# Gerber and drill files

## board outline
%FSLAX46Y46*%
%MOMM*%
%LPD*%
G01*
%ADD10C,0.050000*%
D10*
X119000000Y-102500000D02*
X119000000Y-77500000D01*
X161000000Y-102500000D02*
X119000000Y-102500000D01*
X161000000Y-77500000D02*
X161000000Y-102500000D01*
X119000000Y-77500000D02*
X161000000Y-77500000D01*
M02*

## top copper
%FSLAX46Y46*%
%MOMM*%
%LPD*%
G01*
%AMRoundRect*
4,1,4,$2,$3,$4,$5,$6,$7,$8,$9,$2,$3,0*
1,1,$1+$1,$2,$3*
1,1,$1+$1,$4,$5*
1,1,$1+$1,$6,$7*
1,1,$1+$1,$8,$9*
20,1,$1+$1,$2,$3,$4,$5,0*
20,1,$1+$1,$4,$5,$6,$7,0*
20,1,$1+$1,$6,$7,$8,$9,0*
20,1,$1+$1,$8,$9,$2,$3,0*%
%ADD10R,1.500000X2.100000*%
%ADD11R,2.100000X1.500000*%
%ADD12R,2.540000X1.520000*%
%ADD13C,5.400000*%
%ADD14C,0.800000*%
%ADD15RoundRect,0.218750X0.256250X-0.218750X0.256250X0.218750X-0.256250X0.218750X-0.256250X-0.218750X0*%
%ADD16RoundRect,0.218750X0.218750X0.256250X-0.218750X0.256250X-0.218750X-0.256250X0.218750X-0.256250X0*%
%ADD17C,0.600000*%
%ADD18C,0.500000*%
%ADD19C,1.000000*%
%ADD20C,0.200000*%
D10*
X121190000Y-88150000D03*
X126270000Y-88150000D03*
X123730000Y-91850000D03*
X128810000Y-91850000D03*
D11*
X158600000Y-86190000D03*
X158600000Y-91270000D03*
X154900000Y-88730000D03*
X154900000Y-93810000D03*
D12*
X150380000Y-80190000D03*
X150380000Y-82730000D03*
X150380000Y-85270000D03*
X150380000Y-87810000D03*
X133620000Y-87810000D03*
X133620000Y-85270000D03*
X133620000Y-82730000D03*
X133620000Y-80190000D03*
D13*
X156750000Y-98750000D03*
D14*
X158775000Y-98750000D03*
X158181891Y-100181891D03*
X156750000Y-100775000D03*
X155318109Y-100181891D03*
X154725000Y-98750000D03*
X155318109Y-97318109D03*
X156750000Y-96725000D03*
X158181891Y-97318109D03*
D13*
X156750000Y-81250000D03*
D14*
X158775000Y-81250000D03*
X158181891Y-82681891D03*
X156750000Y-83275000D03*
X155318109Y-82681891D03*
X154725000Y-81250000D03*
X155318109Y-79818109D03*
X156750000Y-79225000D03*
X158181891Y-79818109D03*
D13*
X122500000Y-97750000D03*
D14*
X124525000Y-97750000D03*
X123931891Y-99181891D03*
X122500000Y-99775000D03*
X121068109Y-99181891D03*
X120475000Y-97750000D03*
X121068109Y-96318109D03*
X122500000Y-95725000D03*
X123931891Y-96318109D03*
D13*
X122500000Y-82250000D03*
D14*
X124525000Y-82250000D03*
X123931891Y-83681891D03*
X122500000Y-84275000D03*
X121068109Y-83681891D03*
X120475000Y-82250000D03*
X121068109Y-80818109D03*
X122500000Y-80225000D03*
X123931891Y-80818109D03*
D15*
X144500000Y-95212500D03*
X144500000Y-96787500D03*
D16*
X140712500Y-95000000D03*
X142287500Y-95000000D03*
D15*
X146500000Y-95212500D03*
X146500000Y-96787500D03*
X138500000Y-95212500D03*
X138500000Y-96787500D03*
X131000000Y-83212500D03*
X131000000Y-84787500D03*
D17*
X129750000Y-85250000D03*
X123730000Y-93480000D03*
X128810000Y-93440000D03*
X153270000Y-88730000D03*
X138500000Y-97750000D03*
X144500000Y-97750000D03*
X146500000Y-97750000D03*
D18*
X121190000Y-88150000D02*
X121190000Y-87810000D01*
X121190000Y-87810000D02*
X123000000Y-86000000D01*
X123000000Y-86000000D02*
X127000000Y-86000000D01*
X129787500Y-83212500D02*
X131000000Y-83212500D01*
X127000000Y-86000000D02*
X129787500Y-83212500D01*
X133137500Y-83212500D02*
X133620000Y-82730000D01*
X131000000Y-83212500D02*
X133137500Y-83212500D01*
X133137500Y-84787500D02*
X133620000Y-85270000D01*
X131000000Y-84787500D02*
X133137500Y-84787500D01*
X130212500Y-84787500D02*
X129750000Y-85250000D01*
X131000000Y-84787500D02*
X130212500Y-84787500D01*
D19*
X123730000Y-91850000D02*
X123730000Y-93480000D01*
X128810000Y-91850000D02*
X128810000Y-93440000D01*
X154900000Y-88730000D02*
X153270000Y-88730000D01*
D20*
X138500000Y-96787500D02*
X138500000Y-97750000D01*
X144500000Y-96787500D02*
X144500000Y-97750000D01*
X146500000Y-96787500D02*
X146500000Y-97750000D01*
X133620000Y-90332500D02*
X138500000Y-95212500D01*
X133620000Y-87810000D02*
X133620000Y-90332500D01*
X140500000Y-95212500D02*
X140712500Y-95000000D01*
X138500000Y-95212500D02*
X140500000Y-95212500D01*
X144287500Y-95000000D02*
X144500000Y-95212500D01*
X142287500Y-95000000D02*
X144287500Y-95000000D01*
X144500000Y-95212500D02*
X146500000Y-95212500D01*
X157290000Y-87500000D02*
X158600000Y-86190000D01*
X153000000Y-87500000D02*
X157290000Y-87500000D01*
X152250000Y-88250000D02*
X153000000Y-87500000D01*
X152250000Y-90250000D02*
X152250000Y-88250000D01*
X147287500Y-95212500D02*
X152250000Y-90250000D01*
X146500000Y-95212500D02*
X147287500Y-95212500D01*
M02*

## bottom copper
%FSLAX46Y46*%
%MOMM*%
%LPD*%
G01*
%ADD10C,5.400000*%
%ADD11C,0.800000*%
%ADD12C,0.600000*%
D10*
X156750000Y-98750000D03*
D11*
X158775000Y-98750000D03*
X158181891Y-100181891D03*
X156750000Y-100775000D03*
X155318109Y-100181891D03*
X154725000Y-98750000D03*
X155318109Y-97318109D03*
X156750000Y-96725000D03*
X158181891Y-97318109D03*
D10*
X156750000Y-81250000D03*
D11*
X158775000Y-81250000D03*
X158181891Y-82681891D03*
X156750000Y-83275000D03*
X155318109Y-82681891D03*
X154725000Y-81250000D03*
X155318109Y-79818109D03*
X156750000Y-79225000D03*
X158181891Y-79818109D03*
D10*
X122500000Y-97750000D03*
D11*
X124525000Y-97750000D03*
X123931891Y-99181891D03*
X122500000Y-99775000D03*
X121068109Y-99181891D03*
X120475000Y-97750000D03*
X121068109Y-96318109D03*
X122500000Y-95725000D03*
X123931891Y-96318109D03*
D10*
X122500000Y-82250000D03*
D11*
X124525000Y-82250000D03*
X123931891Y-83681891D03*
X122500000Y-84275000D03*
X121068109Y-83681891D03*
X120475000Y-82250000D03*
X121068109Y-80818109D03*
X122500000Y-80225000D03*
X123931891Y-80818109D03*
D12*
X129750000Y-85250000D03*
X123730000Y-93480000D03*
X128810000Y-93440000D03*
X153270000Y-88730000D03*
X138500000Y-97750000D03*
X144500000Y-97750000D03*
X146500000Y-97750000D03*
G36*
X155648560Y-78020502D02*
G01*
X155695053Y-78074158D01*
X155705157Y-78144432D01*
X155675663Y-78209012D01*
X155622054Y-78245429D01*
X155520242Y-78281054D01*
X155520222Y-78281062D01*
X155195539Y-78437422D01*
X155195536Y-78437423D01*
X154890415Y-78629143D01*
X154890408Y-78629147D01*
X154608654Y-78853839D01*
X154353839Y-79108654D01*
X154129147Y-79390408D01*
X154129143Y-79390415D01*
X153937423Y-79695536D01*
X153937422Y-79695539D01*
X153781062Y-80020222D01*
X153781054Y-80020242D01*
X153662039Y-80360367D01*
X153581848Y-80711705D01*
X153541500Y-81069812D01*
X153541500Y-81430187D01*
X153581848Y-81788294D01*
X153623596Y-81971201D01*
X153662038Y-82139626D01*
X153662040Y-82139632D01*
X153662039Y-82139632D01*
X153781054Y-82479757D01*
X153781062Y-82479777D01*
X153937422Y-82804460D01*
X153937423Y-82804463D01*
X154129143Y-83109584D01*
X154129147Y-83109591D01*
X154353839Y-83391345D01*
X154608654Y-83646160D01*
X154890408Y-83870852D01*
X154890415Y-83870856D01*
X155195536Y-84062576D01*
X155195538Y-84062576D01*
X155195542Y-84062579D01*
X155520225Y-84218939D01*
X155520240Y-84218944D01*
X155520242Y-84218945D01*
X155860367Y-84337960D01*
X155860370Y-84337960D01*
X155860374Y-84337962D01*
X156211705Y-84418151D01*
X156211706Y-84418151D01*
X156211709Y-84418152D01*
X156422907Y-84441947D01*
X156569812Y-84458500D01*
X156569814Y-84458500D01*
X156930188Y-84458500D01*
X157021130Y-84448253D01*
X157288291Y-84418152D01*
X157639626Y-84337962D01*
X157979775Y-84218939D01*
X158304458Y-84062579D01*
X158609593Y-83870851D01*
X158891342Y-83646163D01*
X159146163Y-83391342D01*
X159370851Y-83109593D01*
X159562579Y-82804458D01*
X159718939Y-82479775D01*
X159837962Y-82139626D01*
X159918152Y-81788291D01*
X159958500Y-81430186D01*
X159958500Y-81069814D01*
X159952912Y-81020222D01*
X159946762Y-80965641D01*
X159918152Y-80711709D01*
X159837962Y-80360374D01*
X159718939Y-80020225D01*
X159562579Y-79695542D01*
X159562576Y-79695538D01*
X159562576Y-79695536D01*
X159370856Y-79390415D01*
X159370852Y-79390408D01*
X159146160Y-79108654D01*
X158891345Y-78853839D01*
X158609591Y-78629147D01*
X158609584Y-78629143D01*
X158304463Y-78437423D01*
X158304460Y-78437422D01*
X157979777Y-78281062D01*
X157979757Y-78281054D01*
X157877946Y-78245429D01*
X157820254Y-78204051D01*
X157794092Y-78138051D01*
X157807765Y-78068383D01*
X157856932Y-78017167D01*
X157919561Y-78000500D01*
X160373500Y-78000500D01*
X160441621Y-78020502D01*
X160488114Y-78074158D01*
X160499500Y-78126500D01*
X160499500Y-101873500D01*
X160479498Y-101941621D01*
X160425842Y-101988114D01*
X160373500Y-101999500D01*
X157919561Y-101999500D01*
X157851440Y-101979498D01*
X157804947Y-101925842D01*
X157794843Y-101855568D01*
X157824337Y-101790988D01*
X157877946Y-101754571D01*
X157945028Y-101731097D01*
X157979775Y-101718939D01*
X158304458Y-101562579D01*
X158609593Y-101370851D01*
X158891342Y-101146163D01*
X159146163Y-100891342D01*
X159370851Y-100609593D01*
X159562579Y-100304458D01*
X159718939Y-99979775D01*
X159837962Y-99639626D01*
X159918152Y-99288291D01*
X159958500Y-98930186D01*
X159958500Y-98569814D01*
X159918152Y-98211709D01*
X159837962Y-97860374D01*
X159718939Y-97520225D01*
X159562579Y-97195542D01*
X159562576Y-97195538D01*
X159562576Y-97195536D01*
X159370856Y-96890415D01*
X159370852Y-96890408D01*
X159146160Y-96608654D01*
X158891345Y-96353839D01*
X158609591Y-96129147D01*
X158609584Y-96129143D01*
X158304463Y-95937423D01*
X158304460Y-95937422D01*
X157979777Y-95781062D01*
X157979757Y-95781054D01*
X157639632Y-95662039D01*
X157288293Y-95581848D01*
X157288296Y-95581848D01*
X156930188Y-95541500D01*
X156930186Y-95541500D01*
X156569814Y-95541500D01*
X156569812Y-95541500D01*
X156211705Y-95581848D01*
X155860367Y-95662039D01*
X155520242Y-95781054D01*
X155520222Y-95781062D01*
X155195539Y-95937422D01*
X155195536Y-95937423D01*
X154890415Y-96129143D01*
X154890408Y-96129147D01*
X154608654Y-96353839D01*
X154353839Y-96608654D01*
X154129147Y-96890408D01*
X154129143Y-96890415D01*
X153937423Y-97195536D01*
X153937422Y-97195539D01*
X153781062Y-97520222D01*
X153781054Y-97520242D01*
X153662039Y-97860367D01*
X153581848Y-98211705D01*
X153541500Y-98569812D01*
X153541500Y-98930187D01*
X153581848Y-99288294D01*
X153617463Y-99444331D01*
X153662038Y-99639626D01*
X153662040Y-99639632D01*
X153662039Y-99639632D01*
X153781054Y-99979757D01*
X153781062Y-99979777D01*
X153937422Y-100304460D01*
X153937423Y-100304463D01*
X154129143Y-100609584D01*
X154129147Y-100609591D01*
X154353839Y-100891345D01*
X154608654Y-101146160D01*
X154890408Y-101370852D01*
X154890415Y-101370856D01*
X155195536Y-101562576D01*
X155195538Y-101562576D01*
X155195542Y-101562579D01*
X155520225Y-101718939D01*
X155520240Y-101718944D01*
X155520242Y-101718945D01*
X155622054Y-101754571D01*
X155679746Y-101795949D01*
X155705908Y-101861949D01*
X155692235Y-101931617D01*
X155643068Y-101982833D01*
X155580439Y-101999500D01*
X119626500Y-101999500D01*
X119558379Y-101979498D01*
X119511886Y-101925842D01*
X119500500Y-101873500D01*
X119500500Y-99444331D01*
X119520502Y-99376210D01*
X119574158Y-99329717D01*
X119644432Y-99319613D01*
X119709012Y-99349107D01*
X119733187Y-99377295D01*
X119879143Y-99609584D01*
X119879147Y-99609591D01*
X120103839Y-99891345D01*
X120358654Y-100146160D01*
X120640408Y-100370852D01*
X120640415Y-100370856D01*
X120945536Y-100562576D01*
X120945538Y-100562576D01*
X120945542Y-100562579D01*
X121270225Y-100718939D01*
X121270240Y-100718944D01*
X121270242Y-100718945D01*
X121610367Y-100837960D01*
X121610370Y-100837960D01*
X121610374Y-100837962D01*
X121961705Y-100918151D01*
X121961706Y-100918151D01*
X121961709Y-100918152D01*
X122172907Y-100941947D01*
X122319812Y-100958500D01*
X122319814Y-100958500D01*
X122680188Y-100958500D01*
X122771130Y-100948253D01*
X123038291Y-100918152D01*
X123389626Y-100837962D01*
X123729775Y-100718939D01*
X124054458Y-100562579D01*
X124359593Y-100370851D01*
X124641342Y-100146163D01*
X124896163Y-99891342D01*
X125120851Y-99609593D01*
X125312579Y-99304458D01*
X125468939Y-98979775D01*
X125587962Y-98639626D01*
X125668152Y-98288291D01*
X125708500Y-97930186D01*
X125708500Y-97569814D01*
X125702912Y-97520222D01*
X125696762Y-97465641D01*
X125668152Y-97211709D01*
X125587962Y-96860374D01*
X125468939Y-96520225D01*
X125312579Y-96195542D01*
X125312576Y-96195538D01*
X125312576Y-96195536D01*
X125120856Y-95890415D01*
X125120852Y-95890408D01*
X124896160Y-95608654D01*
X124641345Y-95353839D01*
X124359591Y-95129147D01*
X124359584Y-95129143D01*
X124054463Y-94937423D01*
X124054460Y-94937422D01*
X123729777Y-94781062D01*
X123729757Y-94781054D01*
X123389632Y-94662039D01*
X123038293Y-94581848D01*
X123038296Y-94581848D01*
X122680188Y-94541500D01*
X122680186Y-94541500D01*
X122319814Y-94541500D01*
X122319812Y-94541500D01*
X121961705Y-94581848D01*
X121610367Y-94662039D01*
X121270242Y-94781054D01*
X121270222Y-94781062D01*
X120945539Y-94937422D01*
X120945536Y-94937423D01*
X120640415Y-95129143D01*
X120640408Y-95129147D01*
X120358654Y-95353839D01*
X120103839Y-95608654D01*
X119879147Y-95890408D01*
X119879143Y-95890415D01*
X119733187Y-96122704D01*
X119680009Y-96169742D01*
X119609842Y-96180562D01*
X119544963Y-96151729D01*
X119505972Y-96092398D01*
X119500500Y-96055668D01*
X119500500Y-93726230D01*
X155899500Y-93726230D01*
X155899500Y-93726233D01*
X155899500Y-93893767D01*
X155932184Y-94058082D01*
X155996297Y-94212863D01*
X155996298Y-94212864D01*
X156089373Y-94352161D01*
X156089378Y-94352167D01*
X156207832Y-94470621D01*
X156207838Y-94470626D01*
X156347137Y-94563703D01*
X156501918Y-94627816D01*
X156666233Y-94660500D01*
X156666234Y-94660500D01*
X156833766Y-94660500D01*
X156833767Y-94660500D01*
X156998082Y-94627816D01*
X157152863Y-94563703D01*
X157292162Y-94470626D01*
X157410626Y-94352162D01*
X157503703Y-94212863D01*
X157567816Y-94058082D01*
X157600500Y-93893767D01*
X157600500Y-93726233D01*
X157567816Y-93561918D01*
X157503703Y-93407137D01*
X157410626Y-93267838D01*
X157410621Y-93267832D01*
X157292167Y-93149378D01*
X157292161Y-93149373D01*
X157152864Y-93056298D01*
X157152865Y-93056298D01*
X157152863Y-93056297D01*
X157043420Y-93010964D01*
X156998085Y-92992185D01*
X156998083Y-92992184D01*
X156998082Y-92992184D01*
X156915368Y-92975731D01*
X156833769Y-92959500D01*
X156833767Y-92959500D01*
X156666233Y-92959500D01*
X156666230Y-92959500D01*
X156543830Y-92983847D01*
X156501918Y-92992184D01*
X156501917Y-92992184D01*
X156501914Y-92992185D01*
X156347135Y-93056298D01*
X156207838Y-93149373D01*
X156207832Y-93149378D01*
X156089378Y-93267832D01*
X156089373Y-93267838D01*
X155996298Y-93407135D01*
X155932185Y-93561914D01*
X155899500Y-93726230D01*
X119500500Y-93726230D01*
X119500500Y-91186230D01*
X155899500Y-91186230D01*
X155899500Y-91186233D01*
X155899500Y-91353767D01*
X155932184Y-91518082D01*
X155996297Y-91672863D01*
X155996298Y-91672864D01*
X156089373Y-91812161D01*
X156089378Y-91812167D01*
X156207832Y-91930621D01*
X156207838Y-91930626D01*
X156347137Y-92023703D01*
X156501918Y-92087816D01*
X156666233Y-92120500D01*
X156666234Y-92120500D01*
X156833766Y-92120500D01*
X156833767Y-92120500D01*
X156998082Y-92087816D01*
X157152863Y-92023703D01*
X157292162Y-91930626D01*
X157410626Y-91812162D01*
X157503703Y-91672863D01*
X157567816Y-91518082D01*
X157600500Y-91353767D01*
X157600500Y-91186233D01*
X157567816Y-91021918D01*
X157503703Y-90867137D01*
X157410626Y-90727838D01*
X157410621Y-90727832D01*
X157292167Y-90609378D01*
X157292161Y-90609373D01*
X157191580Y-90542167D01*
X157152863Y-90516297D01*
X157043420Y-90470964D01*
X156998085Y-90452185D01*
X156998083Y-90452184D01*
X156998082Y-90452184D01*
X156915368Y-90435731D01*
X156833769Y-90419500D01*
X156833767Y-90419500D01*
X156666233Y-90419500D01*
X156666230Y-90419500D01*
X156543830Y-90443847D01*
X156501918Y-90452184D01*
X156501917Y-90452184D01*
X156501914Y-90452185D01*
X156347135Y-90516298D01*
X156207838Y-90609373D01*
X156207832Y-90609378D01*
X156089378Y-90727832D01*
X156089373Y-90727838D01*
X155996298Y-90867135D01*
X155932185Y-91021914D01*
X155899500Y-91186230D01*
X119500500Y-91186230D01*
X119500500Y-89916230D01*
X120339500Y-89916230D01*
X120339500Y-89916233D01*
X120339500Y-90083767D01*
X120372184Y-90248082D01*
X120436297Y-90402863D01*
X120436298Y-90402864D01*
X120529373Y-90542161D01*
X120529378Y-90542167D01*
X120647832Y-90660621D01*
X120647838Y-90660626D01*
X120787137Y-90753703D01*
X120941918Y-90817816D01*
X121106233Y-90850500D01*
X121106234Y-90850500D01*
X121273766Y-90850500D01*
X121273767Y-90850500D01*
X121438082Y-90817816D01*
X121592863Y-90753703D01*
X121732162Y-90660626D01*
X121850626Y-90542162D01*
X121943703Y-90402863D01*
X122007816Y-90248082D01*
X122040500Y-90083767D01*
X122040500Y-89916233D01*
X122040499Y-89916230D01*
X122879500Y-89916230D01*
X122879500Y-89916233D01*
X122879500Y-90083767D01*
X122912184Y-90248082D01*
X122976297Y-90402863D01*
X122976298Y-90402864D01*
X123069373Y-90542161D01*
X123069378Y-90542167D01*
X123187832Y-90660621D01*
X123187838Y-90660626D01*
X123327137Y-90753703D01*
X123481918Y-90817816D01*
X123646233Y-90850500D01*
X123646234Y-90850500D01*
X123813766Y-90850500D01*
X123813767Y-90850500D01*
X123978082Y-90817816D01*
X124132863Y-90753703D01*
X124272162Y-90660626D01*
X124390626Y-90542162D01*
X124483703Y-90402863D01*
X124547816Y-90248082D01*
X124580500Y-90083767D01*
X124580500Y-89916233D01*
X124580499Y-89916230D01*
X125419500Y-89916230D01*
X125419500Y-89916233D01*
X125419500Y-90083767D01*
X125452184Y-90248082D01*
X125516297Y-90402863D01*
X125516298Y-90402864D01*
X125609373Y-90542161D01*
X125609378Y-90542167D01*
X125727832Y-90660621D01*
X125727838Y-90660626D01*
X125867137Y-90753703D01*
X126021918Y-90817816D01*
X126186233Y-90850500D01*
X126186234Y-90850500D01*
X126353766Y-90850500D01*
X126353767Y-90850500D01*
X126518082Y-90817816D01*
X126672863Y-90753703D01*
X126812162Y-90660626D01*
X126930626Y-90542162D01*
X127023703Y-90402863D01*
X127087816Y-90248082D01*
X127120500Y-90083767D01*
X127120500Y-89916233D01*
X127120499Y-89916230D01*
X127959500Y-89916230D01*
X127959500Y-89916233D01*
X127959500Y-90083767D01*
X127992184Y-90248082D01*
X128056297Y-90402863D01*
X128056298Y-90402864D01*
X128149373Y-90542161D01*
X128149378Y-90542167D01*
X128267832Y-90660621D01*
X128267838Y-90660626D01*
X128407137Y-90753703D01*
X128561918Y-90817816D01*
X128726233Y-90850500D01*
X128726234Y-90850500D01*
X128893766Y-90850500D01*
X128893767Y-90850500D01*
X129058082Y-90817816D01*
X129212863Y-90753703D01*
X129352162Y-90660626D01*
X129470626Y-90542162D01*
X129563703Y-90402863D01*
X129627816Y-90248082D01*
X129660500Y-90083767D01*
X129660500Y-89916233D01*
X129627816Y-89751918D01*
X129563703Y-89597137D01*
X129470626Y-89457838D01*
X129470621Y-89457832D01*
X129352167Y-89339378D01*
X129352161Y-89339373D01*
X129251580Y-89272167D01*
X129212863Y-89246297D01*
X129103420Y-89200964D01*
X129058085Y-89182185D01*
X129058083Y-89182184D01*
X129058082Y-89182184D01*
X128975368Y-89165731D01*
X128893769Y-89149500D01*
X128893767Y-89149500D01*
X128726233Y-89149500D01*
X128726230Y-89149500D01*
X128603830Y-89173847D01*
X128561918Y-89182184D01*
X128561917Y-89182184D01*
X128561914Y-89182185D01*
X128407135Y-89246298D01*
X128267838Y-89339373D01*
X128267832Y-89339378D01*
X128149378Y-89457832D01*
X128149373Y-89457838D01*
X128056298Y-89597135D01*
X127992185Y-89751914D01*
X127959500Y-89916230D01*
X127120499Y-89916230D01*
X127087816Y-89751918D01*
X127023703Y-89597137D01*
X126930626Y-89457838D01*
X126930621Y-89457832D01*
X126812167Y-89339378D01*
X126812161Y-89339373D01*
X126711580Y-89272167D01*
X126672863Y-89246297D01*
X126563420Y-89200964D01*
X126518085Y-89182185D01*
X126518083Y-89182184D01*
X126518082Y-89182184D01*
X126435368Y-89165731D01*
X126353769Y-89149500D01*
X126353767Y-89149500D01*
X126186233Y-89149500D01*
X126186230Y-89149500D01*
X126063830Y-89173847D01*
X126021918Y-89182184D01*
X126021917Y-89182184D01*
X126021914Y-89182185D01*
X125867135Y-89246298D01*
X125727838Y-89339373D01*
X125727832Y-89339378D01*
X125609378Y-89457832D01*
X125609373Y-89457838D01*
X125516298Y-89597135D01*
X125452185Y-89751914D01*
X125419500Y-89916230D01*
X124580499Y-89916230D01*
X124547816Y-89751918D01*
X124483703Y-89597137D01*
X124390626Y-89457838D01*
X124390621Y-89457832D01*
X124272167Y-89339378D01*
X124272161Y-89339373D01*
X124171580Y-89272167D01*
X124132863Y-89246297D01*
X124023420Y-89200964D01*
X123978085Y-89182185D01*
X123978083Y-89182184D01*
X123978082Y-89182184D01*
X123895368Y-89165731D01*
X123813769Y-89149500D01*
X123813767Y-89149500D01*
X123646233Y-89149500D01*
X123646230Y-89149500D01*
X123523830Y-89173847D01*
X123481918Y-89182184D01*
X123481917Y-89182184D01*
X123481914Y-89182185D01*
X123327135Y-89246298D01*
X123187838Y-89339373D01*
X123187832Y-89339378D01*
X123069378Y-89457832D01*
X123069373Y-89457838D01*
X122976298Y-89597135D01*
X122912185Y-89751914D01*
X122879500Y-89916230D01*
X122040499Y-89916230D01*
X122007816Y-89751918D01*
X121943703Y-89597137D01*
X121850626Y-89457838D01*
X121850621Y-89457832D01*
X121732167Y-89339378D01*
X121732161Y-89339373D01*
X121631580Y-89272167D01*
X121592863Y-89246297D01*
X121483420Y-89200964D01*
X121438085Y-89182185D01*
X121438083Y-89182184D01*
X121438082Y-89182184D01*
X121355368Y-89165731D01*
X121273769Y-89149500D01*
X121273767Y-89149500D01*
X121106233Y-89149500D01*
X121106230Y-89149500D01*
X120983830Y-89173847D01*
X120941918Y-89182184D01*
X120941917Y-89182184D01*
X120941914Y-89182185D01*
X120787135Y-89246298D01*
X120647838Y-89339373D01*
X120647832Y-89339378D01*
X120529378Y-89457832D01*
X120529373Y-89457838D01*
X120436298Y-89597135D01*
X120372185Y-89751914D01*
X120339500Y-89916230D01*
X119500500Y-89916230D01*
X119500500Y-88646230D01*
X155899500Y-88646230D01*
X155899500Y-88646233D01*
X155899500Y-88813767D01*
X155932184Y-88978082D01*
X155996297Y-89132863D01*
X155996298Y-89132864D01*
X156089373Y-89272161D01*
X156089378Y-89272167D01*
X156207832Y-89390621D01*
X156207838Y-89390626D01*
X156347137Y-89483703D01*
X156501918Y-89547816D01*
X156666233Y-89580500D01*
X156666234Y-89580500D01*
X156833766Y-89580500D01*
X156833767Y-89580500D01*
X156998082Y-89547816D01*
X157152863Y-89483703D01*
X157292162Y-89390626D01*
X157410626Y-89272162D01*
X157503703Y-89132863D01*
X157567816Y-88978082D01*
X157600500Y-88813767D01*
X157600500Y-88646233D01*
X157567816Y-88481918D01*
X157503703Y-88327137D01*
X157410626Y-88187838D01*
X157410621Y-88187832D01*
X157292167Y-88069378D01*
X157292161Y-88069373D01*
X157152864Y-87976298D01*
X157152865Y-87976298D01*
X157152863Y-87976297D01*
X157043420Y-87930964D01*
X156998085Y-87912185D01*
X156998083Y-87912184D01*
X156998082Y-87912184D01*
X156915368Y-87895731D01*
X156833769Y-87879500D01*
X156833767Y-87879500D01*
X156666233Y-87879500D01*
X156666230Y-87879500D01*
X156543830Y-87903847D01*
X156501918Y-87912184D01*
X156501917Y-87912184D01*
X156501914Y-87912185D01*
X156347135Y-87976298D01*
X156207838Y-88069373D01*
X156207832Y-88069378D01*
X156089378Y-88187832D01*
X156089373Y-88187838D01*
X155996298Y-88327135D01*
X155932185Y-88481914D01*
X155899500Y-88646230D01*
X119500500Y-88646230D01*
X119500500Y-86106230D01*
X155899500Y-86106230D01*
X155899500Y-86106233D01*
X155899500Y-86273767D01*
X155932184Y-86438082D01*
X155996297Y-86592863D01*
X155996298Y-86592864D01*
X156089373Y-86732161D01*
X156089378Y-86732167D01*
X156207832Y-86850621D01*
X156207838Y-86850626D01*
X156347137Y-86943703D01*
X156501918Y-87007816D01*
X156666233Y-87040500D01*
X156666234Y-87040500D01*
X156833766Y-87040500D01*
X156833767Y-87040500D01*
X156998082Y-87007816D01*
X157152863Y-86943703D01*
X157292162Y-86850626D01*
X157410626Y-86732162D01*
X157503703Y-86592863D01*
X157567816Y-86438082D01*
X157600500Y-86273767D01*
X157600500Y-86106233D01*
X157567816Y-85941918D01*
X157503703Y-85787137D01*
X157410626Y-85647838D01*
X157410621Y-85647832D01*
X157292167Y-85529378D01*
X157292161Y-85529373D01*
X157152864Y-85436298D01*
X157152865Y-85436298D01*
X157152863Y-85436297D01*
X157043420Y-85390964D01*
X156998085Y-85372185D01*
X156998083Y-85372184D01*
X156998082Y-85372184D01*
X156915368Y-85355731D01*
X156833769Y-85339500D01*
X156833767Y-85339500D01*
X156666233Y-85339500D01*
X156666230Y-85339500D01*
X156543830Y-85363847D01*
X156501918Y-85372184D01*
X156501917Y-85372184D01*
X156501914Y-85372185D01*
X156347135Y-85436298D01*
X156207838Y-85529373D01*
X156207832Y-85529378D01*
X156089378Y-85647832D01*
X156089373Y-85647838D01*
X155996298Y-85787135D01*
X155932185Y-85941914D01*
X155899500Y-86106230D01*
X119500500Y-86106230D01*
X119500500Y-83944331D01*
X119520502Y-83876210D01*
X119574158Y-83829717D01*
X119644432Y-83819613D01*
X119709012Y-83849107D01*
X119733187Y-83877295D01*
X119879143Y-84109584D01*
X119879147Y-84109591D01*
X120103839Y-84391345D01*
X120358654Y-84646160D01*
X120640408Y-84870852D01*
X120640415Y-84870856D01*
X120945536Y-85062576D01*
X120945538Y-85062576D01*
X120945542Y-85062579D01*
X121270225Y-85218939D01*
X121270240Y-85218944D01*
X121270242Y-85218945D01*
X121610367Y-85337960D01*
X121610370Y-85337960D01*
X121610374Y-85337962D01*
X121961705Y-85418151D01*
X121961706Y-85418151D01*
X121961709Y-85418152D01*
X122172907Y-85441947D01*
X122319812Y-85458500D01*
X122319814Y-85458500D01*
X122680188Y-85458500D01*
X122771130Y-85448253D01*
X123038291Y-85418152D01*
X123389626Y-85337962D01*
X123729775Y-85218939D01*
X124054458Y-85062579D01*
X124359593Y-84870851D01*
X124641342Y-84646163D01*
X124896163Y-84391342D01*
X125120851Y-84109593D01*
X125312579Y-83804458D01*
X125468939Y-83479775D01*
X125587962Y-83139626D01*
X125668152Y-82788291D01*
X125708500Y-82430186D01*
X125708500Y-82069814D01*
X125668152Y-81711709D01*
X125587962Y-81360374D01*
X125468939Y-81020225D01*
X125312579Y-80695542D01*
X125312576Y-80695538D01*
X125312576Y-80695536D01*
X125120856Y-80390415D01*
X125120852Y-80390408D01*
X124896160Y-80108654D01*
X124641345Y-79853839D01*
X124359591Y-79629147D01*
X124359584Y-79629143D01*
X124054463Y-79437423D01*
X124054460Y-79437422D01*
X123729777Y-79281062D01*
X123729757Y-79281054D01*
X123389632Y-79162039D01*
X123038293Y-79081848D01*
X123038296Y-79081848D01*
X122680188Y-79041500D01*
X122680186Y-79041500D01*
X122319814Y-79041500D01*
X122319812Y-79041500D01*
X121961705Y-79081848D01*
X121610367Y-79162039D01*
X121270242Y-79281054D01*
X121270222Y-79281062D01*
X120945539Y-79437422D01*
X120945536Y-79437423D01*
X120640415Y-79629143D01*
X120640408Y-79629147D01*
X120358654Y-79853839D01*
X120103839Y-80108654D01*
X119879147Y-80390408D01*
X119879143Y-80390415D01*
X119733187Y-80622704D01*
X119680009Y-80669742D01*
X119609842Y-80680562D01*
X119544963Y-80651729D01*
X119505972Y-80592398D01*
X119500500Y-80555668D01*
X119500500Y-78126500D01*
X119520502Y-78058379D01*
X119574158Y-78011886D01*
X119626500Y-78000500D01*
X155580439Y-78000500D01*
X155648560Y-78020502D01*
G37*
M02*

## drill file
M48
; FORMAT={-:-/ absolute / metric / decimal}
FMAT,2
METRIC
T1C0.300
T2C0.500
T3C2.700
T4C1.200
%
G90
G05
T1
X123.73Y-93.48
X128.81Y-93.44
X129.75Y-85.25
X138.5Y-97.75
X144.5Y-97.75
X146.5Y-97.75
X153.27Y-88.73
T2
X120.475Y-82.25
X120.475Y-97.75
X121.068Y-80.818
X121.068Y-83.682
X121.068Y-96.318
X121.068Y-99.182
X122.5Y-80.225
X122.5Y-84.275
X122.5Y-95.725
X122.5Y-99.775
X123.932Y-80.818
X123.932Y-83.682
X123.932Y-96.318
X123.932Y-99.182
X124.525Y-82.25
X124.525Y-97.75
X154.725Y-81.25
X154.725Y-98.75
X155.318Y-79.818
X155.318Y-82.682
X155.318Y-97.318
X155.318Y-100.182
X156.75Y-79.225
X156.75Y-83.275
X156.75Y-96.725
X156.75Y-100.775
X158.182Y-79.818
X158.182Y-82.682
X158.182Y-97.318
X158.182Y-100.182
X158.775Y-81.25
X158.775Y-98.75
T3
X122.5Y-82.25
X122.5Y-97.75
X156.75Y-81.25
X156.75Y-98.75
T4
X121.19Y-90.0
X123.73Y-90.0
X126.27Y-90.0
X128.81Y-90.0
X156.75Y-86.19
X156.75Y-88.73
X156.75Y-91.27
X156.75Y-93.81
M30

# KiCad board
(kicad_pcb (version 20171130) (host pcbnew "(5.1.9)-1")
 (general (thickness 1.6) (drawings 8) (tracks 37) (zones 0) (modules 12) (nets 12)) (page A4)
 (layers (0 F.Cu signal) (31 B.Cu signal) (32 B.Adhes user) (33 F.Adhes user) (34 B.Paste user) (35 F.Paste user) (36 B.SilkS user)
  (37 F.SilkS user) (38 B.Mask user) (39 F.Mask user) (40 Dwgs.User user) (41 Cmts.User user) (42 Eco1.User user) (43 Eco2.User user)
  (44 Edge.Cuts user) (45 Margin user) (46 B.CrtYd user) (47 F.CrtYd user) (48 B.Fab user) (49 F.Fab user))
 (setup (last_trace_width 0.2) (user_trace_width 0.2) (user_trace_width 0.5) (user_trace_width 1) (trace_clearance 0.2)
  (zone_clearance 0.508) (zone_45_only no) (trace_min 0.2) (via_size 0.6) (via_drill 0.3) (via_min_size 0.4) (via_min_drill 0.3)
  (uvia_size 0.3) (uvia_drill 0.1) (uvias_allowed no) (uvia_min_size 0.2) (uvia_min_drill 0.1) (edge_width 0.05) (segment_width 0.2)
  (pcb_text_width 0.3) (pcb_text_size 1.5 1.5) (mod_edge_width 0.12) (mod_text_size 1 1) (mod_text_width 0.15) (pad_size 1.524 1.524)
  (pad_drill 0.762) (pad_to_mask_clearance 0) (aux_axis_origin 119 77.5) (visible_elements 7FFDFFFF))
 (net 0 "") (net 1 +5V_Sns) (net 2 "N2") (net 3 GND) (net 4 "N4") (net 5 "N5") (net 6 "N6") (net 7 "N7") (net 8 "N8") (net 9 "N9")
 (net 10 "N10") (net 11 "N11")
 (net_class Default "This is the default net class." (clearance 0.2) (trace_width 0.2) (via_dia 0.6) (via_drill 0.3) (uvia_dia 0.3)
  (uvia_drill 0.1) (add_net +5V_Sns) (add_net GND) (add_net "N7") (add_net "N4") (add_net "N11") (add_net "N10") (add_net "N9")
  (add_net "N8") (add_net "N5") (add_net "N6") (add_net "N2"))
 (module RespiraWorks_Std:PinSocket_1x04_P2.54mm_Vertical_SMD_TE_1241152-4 (layer F.Cu) (at 125 90 90)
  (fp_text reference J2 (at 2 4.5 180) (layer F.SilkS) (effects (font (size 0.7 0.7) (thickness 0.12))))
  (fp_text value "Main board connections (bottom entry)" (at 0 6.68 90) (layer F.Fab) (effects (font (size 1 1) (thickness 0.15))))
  (pad "" np_thru_hole circle (at 0 1.27 90) (size 1.2 1.2) (drill 1.2) (layers *.Cu *.Mask))
  (pad "" np_thru_hole circle (at 0 -1.27 90) (size 1.2 1.2) (drill 1.2) (layers *.Cu *.Mask))
  (pad "" np_thru_hole circle (at 0 -3.81 90) (size 1.2 1.2) (drill 1.2) (layers *.Cu *.Mask))
  (pad 1 smd rect (at 1.85 -3.81 90) (size 2.1 1.5) (layers F.Cu F.Paste F.Mask) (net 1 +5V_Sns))
  (pad 3 smd rect (at 1.85 1.27 90) (size 2.1 1.5) (layers F.Cu F.Paste F.Mask) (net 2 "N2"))
  (pad 2 smd rect (at -1.85 -1.27 90) (size 2.1 1.5) (layers F.Cu F.Paste F.Mask) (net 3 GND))
  (pad 4 smd rect (at -1.85 3.81 90) (size 2.1 1.5) (layers F.Cu F.Paste F.Mask) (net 3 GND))
  (pad "" np_thru_hole circle (at 0 3.81 90) (size 1.2 1.2) (drill 1.2) (layers *.Cu *.Mask)))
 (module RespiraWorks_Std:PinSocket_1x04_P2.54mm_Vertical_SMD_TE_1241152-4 (layer F.Cu) (at 156.75 90)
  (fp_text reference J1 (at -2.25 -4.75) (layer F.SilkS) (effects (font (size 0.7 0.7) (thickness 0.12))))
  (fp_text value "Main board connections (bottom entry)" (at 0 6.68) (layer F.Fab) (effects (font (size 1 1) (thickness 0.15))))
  (pad "" np_thru_hole circle (at 0 1.27) (size 1.2 1.2) (drill 1.2) (layers *.Cu *.Mask))
  (pad "" np_thru_hole circle (at 0 -1.27) (size 1.2 1.2) (drill 1.2) (layers *.Cu *.Mask))
  (pad "" np_thru_hole circle (at 0 -3.81) (size 1.2 1.2) (drill 1.2) (layers *.Cu *.Mask))
  (pad 1 smd rect (at 1.85 -3.81) (size 2.1 1.5) (layers F.Cu F.Paste F.Mask) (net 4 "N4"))
  (pad 3 smd rect (at 1.85 1.27) (size 2.1 1.5) (layers F.Cu F.Paste F.Mask) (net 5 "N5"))
  (pad 2 smd rect (at -1.85 -1.27) (size 2.1 1.5) (layers F.Cu F.Paste F.Mask) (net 3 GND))
  (pad 4 smd rect (at -1.85 3.81) (size 2.1 1.5) (layers F.Cu F.Paste F.Mask) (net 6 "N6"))
  (pad "" np_thru_hole circle (at 0 3.81) (size 1.2 1.2) (drill 1.2) (layers *.Cu *.Mask)))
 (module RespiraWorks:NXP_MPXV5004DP (layer F.Cu) (at 142 84)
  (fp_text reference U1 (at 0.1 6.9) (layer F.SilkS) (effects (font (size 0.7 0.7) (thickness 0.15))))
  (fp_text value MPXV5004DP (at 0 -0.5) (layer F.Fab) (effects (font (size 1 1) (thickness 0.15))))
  (pad 8 smd rect (at 8.38 -3.81) (size 2.54 1.52) (layers F.Cu F.Paste F.Mask))
  (pad 7 smd rect (at 8.38 -1.27) (size 2.54 1.52) (layers F.Cu F.Paste F.Mask))
  (pad 6 smd rect (at 8.38 1.27) (size 2.54 1.52) (layers F.Cu F.Paste F.Mask))
  (pad 5 smd rect (at 8.38 3.81) (size 2.54 1.52) (layers F.Cu F.Paste F.Mask))
  (pad 4 smd rect (at -8.38 3.81) (size 2.54 1.52) (layers F.Cu F.Paste F.Mask) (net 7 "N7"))
  (pad 3 smd rect (at -8.38 1.27) (size 2.54 1.52) (layers F.Cu F.Paste F.Mask) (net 3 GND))
  (pad 2 smd rect (at -8.38 -1.27) (size 2.54 1.52) (layers F.Cu F.Paste F.Mask) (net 1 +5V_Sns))
  (pad 1 smd rect (at -8.38 -3.81) (size 2.54 1.52) (layers F.Cu F.Paste F.Mask)))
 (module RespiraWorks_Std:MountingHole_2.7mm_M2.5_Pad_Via (layer F.Cu) (at 156.75 98.75)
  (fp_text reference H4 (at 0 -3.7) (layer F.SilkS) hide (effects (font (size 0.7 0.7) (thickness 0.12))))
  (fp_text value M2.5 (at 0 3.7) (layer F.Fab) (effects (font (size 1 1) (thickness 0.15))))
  (pad 1 thru_hole circle (at 0 0) (size 5.4 5.4) (drill 2.7) (layers *.Cu *.Mask) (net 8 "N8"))
  (pad 1 thru_hole circle (at 2.025 0) (size 0.8 0.8) (drill 0.5) (layers *.Cu *.Mask) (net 8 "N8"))
  (pad 1 thru_hole circle (at 1.431891 1.431891) (size 0.8 0.8) (drill 0.5) (layers *.Cu *.Mask) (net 8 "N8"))
  (pad 1 thru_hole circle (at 0 2.025) (size 0.8 0.8) (drill 0.5) (layers *.Cu *.Mask) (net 8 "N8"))
  (pad 1 thru_hole circle (at -1.431891 1.431891) (size 0.8 0.8) (drill 0.5) (layers *.Cu *.Mask) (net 8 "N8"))
  (pad 1 thru_hole circle (at -2.025 0) (size 0.8 0.8) (drill 0.5) (layers *.Cu *.Mask) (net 8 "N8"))
  (pad 1 thru_hole circle (at -1.431891 -1.431891) (size 0.8 0.8) (drill 0.5) (layers *.Cu *.Mask) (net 8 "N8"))
  (pad 1 thru_hole circle (at 0 -2.025) (size 0.8 0.8) (drill 0.5) (layers *.Cu *.Mask) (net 8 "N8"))
  (pad 1 thru_hole circle (at 1.431891 -1.431891) (size 0.8 0.8) (drill 0.5) (layers *.Cu *.Mask) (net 8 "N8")))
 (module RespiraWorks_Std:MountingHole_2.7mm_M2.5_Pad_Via (layer F.Cu) (at 156.75 81.25)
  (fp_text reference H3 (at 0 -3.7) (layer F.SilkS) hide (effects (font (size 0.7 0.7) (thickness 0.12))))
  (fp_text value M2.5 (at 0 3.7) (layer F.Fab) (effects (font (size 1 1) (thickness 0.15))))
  (pad 1 thru_hole circle (at 0 0) (size 5.4 5.4) (drill 2.7) (layers *.Cu *.Mask) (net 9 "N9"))
  (pad 1 thru_hole circle (at 2.025 0) (size 0.8 0.8) (drill 0.5) (layers *.Cu *.Mask) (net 9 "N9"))
  (pad 1 thru_hole circle (at 1.431891 1.431891) (size 0.8 0.8) (drill 0.5) (layers *.Cu *.Mask) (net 9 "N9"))
  (pad 1 thru_hole circle (at 0 2.025) (size 0.8 0.8) (drill 0.5) (layers *.Cu *.Mask) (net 9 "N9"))
  (pad 1 thru_hole circle (at -1.431891 1.431891) (size 0.8 0.8) (drill 0.5) (layers *.Cu *.Mask) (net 9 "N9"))
  (pad 1 thru_hole circle (at -2.025 0) (size 0.8 0.8) (drill 0.5) (layers *.Cu *.Mask) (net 9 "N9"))
  (pad 1 thru_hole circle (at -1.431891 -1.431891) (size 0.8 0.8) (drill 0.5) (layers *.Cu *.Mask) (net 9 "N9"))
  (pad 1 thru_hole circle (at 0 -2.025) (size 0.8 0.8) (drill 0.5) (layers *.Cu *.Mask) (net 9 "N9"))
  (pad 1 thru_hole circle (at 1.431891 -1.431891) (size 0.8 0.8) (drill 0.5) (layers *.Cu *.Mask) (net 9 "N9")))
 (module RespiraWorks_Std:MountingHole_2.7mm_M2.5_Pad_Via (layer F.Cu) (at 122.5 97.75)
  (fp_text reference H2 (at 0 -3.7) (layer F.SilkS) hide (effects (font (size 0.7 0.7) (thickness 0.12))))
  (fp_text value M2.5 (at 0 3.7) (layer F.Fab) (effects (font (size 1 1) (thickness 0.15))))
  (pad 1 thru_hole circle (at 0 0) (size 5.4 5.4) (drill 2.7) (layers *.Cu *.Mask) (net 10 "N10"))
  (pad 1 thru_hole circle (at 2.025 0) (size 0.8 0.8) (drill 0.5) (layers *.Cu *.Mask) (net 10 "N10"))
  (pad 1 thru_hole circle (at 1.431891 1.431891) (size 0.8 0.8) (drill 0.5) (layers *.Cu *.Mask) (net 10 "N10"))
  (pad 1 thru_hole circle (at 0 2.025) (size 0.8 0.8) (drill 0.5) (layers *.Cu *.Mask) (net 10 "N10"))
  (pad 1 thru_hole circle (at -1.431891 1.431891) (size 0.8 0.8) (drill 0.5) (layers *.Cu *.Mask) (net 10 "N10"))
  (pad 1 thru_hole circle (at -2.025 0) (size 0.8 0.8) (drill 0.5) (layers *.Cu *.Mask) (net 10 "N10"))
  (pad 1 thru_hole circle (at -1.431891 -1.431891) (size 0.8 0.8) (drill 0.5) (layers *.Cu *.Mask) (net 10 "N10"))
  (pad 1 thru_hole circle (at 0 -2.025) (size 0.8 0.8) (drill 0.5) (layers *.Cu *.Mask) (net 10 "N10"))
  (pad 1 thru_hole circle (at 1.431891 -1.431891) (size 0.8 0.8) (drill 0.5) (layers *.Cu *.Mask) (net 10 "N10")))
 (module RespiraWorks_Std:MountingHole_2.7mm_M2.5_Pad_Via (layer F.Cu) (at 122.5 82.25)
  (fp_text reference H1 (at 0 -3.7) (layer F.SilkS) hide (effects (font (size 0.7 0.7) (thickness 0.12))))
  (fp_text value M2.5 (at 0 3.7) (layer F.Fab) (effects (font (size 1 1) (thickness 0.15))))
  (pad 1 thru_hole circle (at 0 0) (size 5.4 5.4) (drill 2.7) (layers *.Cu *.Mask) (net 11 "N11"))
  (pad 1 thru_hole circle (at 2.025 0) (size 0.8 0.8) (drill 0.5) (layers *.Cu *.Mask) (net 11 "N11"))
  (pad 1 thru_hole circle (at 1.431891 1.431891) (size 0.8 0.8) (drill 0.5) (layers *.Cu *.Mask) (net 11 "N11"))
  (pad 1 thru_hole circle (at 0 2.025) (size 0.8 0.8) (drill 0.5) (layers *.Cu *.Mask) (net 11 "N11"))
  (pad 1 thru_hole circle (at -1.431891 1.431891) (size 0.8 0.8) (drill 0.5) (layers *.Cu *.Mask) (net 11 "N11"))
  (pad 1 thru_hole circle (at -2.025 0) (size 0.8 0.8) (drill 0.5) (layers *.Cu *.Mask) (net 11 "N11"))
  (pad 1 thru_hole circle (at -1.431891 -1.431891) (size 0.8 0.8) (drill 0.5) (layers *.Cu *.Mask) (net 11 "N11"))
  (pad 1 thru_hole circle (at 0 -2.025) (size 0.8 0.8) (drill 0.5) (layers *.Cu *.Mask) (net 11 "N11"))
  (pad 1 thru_hole circle (at 1.431891 -1.431891) (size 0.8 0.8) (drill 0.5) (layers *.Cu *.Mask) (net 11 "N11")))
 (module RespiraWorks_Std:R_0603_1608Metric (layer F.Cu) (at 144.5 96 90)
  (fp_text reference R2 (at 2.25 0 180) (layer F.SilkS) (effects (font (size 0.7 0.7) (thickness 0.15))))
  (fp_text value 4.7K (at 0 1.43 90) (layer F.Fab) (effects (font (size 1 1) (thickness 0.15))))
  (pad 2 smd roundrect (at 0.7875 0 90) (size 0.875 0.95) (layers F.Cu F.Paste F.Mask) (roundrect_rratio 0.25) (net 4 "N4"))
  (pad 1 smd roundrect (at -0.7875 0 90) (size 0.875 0.95) (layers F.Cu F.Paste F.Mask) (roundrect_rratio 0.25) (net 3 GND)))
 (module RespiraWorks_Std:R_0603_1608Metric (layer F.Cu) (at 141.5 95 180)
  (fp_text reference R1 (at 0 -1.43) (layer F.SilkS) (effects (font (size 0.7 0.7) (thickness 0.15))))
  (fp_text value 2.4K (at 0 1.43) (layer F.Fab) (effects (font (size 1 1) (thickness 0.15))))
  (pad 2 smd roundrect (at 0.7875 0 180) (size 0.875 0.95) (layers F.Cu F.Paste F.Mask) (roundrect_rratio 0.25) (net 7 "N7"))
  (pad 1 smd roundrect (at -0.7875 0 180) (size 0.875 0.95) (layers F.Cu F.Paste F.Mask) (roundrect_rratio 0.25) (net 4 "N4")))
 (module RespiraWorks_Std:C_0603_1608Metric (layer F.Cu) (at 146.5 96 90)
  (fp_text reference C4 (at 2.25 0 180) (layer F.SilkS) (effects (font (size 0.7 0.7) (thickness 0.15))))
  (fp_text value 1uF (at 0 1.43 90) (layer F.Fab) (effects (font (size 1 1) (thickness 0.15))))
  (pad 2 smd roundrect (at 0.7875 0 90) (size 0.875 0.95) (layers F.Cu F.Paste F.Mask) (roundrect_rratio 0.25) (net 4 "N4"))
  (pad 1 smd roundrect (at -0.7875 0 90) (size 0.875 0.95) (layers F.Cu F.Paste F.Mask) (roundrect_rratio 0.25) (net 3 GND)))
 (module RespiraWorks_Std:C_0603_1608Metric (layer F.Cu) (at 138.5 96 90)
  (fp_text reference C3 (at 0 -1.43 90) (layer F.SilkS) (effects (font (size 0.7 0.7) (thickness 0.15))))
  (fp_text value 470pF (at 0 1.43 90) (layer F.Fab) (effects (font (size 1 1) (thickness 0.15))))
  (pad 2 smd roundrect (at 0.7875 0 90) (size 0.875 0.95) (layers F.Cu F.Paste F.Mask) (roundrect_rratio 0.25) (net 7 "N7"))
  (pad 1 smd roundrect (at -0.7875 0 90) (size 0.875 0.95) (layers F.Cu F.Paste F.Mask) (roundrect_rratio 0.25) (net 3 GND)))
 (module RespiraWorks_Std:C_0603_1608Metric (layer F.Cu) (at 131 84 90)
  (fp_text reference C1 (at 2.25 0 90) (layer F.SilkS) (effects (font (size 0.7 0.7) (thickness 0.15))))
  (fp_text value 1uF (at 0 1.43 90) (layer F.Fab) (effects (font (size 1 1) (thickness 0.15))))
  (pad 2 smd roundrect (at 0.7875 0 90) (size 0.875 0.95) (layers F.Cu F.Paste F.Mask) (roundrect_rratio 0.25) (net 1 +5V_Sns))
  (pad 1 smd roundrect (at -0.7875 0 90) (size 0.875 0.95) (layers F.Cu F.Paste F.Mask) (roundrect_rratio 0.25) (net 3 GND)))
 (gr_line (start 119 102.5) (end 119 77.5) (layer Edge.Cuts) (width 0.05))
 (gr_line (start 161 102.5) (end 119 102.5) (layer Edge.Cuts) (width 0.05))
 (gr_line (start 161 77.5) (end 161 102.5) (layer Edge.Cuts) (width 0.05))
 (gr_line (start 119 77.5) (end 161 77.5) (layer Edge.Cuts) (width 0.05))
 (segment (start 121.19 88.15) (end 121.19 87.81) (width 0.5) (layer F.Cu) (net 1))
 (segment (start 121.19 87.81) (end 123 86) (width 0.5) (layer F.Cu) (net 1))
 (segment (start 123 86) (end 127 86) (width 0.5) (layer F.Cu) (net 1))
 (segment (start 129.7875 83.2125) (end 131 83.2125) (width 0.5) (layer F.Cu) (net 1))
 (segment (start 127 86) (end 129.7875 83.2125) (width 0.5) (layer F.Cu) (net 1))
 (segment (start 133.1375 83.2125) (end 133.62 82.73) (width 0.5) (layer F.Cu) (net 1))
 (segment (start 131 83.2125) (end 133.1375 83.2125) (width 0.5) (layer F.Cu) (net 1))
 (segment (start 133.1375 84.7875) (end 133.62 85.27) (width 0.5) (layer F.Cu) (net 3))
 (segment (start 131 84.7875) (end 133.1375 84.7875) (width 0.5) (layer F.Cu) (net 3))
 (via (at 129.75 85.25) (size 0.6) (drill 0.3) (layers F.Cu B.Cu) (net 3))
 (segment (start 130.2125 84.7875) (end 129.75 85.25) (width 0.5) (layer F.Cu) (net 3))
 (segment (start 131 84.7875) (end 130.2125 84.7875) (width 0.5) (layer F.Cu) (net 3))
 (segment (start 123.73 91.85) (end 123.73 93.48) (width 1) (layer F.Cu) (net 3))
 (via (at 123.73 93.48) (size 0.6) (drill 0.3) (layers F.Cu B.Cu) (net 3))
 (segment (start 128.81 91.85) (end 128.81 93.44) (width 1) (layer F.Cu) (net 3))
 (via (at 128.81 93.44) (size 0.6) (drill 0.3) (layers F.Cu B.Cu) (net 3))
 (segment (start 154.9 88.73) (end 153.27 88.73) (width 1) (layer F.Cu) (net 3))
 (via (at 153.27 88.73) (size 0.6) (drill 0.3) (layers F.Cu B.Cu) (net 3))
 (segment (start 138.5 96.7875) (end 138.5 97.75) (width 0.2) (layer F.Cu) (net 3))
 (via (at 138.5 97.75) (size 0.6) (drill 0.3) (layers F.Cu B.Cu) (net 3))
 (segment (start 144.5 96.7875) (end 144.5 97.75) (width 0.2) (layer F.Cu) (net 3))
 (via (at 144.5 97.75) (size 0.6) (drill 0.3) (layers F.Cu B.Cu) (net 3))
 (segment (start 146.5 96.7875) (end 146.5 97.75) (width 0.2) (layer F.Cu) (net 3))
 (via (at 146.5 97.75) (size 0.6) (drill 0.3) (layers F.Cu B.Cu) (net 3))
 (segment (start 133.62 90.3325) (end 138.5 95.2125) (width 0.2) (layer F.Cu) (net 7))
 (segment (start 133.62 87.81) (end 133.62 90.3325) (width 0.2) (layer F.Cu) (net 7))
 (segment (start 140.5 95.2125) (end 140.7125 95) (width 0.2) (layer F.Cu) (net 7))
 (segment (start 138.5 95.2125) (end 140.5 95.2125) (width 0.2) (layer F.Cu) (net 7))
 (segment (start 144.2875 95) (end 144.5 95.2125) (width 0.2) (layer F.Cu) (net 4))
 (segment (start 142.2875 95) (end 144.2875 95) (width 0.2) (layer F.Cu) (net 4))
 (segment (start 144.5 95.2125) (end 146.5 95.2125) (width 0.2) (layer F.Cu) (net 4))
 (segment (start 157.29 87.5) (end 158.6 86.19) (width 0.2) (layer F.Cu) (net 4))
 (segment (start 153 87.5) (end 157.29 87.5) (width 0.2) (layer F.Cu) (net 4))
 (segment (start 152.25 88.25) (end 153 87.5) (width 0.2) (layer F.Cu) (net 4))
 (segment (start 152.25 90.25) (end 152.25 88.25) (width 0.2) (layer F.Cu) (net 4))
 (segment (start 147.2875 95.2125) (end 152.25 90.25) (width 0.2) (layer F.Cu) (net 4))
 (segment (start 146.5 95.2125) (end 147.2875 95.2125) (width 0.2) (layer F.Cu) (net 4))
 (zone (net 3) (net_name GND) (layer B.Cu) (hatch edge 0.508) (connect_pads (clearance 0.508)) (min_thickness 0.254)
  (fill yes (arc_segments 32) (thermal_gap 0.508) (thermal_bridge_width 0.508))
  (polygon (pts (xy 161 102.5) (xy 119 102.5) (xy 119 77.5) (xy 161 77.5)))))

